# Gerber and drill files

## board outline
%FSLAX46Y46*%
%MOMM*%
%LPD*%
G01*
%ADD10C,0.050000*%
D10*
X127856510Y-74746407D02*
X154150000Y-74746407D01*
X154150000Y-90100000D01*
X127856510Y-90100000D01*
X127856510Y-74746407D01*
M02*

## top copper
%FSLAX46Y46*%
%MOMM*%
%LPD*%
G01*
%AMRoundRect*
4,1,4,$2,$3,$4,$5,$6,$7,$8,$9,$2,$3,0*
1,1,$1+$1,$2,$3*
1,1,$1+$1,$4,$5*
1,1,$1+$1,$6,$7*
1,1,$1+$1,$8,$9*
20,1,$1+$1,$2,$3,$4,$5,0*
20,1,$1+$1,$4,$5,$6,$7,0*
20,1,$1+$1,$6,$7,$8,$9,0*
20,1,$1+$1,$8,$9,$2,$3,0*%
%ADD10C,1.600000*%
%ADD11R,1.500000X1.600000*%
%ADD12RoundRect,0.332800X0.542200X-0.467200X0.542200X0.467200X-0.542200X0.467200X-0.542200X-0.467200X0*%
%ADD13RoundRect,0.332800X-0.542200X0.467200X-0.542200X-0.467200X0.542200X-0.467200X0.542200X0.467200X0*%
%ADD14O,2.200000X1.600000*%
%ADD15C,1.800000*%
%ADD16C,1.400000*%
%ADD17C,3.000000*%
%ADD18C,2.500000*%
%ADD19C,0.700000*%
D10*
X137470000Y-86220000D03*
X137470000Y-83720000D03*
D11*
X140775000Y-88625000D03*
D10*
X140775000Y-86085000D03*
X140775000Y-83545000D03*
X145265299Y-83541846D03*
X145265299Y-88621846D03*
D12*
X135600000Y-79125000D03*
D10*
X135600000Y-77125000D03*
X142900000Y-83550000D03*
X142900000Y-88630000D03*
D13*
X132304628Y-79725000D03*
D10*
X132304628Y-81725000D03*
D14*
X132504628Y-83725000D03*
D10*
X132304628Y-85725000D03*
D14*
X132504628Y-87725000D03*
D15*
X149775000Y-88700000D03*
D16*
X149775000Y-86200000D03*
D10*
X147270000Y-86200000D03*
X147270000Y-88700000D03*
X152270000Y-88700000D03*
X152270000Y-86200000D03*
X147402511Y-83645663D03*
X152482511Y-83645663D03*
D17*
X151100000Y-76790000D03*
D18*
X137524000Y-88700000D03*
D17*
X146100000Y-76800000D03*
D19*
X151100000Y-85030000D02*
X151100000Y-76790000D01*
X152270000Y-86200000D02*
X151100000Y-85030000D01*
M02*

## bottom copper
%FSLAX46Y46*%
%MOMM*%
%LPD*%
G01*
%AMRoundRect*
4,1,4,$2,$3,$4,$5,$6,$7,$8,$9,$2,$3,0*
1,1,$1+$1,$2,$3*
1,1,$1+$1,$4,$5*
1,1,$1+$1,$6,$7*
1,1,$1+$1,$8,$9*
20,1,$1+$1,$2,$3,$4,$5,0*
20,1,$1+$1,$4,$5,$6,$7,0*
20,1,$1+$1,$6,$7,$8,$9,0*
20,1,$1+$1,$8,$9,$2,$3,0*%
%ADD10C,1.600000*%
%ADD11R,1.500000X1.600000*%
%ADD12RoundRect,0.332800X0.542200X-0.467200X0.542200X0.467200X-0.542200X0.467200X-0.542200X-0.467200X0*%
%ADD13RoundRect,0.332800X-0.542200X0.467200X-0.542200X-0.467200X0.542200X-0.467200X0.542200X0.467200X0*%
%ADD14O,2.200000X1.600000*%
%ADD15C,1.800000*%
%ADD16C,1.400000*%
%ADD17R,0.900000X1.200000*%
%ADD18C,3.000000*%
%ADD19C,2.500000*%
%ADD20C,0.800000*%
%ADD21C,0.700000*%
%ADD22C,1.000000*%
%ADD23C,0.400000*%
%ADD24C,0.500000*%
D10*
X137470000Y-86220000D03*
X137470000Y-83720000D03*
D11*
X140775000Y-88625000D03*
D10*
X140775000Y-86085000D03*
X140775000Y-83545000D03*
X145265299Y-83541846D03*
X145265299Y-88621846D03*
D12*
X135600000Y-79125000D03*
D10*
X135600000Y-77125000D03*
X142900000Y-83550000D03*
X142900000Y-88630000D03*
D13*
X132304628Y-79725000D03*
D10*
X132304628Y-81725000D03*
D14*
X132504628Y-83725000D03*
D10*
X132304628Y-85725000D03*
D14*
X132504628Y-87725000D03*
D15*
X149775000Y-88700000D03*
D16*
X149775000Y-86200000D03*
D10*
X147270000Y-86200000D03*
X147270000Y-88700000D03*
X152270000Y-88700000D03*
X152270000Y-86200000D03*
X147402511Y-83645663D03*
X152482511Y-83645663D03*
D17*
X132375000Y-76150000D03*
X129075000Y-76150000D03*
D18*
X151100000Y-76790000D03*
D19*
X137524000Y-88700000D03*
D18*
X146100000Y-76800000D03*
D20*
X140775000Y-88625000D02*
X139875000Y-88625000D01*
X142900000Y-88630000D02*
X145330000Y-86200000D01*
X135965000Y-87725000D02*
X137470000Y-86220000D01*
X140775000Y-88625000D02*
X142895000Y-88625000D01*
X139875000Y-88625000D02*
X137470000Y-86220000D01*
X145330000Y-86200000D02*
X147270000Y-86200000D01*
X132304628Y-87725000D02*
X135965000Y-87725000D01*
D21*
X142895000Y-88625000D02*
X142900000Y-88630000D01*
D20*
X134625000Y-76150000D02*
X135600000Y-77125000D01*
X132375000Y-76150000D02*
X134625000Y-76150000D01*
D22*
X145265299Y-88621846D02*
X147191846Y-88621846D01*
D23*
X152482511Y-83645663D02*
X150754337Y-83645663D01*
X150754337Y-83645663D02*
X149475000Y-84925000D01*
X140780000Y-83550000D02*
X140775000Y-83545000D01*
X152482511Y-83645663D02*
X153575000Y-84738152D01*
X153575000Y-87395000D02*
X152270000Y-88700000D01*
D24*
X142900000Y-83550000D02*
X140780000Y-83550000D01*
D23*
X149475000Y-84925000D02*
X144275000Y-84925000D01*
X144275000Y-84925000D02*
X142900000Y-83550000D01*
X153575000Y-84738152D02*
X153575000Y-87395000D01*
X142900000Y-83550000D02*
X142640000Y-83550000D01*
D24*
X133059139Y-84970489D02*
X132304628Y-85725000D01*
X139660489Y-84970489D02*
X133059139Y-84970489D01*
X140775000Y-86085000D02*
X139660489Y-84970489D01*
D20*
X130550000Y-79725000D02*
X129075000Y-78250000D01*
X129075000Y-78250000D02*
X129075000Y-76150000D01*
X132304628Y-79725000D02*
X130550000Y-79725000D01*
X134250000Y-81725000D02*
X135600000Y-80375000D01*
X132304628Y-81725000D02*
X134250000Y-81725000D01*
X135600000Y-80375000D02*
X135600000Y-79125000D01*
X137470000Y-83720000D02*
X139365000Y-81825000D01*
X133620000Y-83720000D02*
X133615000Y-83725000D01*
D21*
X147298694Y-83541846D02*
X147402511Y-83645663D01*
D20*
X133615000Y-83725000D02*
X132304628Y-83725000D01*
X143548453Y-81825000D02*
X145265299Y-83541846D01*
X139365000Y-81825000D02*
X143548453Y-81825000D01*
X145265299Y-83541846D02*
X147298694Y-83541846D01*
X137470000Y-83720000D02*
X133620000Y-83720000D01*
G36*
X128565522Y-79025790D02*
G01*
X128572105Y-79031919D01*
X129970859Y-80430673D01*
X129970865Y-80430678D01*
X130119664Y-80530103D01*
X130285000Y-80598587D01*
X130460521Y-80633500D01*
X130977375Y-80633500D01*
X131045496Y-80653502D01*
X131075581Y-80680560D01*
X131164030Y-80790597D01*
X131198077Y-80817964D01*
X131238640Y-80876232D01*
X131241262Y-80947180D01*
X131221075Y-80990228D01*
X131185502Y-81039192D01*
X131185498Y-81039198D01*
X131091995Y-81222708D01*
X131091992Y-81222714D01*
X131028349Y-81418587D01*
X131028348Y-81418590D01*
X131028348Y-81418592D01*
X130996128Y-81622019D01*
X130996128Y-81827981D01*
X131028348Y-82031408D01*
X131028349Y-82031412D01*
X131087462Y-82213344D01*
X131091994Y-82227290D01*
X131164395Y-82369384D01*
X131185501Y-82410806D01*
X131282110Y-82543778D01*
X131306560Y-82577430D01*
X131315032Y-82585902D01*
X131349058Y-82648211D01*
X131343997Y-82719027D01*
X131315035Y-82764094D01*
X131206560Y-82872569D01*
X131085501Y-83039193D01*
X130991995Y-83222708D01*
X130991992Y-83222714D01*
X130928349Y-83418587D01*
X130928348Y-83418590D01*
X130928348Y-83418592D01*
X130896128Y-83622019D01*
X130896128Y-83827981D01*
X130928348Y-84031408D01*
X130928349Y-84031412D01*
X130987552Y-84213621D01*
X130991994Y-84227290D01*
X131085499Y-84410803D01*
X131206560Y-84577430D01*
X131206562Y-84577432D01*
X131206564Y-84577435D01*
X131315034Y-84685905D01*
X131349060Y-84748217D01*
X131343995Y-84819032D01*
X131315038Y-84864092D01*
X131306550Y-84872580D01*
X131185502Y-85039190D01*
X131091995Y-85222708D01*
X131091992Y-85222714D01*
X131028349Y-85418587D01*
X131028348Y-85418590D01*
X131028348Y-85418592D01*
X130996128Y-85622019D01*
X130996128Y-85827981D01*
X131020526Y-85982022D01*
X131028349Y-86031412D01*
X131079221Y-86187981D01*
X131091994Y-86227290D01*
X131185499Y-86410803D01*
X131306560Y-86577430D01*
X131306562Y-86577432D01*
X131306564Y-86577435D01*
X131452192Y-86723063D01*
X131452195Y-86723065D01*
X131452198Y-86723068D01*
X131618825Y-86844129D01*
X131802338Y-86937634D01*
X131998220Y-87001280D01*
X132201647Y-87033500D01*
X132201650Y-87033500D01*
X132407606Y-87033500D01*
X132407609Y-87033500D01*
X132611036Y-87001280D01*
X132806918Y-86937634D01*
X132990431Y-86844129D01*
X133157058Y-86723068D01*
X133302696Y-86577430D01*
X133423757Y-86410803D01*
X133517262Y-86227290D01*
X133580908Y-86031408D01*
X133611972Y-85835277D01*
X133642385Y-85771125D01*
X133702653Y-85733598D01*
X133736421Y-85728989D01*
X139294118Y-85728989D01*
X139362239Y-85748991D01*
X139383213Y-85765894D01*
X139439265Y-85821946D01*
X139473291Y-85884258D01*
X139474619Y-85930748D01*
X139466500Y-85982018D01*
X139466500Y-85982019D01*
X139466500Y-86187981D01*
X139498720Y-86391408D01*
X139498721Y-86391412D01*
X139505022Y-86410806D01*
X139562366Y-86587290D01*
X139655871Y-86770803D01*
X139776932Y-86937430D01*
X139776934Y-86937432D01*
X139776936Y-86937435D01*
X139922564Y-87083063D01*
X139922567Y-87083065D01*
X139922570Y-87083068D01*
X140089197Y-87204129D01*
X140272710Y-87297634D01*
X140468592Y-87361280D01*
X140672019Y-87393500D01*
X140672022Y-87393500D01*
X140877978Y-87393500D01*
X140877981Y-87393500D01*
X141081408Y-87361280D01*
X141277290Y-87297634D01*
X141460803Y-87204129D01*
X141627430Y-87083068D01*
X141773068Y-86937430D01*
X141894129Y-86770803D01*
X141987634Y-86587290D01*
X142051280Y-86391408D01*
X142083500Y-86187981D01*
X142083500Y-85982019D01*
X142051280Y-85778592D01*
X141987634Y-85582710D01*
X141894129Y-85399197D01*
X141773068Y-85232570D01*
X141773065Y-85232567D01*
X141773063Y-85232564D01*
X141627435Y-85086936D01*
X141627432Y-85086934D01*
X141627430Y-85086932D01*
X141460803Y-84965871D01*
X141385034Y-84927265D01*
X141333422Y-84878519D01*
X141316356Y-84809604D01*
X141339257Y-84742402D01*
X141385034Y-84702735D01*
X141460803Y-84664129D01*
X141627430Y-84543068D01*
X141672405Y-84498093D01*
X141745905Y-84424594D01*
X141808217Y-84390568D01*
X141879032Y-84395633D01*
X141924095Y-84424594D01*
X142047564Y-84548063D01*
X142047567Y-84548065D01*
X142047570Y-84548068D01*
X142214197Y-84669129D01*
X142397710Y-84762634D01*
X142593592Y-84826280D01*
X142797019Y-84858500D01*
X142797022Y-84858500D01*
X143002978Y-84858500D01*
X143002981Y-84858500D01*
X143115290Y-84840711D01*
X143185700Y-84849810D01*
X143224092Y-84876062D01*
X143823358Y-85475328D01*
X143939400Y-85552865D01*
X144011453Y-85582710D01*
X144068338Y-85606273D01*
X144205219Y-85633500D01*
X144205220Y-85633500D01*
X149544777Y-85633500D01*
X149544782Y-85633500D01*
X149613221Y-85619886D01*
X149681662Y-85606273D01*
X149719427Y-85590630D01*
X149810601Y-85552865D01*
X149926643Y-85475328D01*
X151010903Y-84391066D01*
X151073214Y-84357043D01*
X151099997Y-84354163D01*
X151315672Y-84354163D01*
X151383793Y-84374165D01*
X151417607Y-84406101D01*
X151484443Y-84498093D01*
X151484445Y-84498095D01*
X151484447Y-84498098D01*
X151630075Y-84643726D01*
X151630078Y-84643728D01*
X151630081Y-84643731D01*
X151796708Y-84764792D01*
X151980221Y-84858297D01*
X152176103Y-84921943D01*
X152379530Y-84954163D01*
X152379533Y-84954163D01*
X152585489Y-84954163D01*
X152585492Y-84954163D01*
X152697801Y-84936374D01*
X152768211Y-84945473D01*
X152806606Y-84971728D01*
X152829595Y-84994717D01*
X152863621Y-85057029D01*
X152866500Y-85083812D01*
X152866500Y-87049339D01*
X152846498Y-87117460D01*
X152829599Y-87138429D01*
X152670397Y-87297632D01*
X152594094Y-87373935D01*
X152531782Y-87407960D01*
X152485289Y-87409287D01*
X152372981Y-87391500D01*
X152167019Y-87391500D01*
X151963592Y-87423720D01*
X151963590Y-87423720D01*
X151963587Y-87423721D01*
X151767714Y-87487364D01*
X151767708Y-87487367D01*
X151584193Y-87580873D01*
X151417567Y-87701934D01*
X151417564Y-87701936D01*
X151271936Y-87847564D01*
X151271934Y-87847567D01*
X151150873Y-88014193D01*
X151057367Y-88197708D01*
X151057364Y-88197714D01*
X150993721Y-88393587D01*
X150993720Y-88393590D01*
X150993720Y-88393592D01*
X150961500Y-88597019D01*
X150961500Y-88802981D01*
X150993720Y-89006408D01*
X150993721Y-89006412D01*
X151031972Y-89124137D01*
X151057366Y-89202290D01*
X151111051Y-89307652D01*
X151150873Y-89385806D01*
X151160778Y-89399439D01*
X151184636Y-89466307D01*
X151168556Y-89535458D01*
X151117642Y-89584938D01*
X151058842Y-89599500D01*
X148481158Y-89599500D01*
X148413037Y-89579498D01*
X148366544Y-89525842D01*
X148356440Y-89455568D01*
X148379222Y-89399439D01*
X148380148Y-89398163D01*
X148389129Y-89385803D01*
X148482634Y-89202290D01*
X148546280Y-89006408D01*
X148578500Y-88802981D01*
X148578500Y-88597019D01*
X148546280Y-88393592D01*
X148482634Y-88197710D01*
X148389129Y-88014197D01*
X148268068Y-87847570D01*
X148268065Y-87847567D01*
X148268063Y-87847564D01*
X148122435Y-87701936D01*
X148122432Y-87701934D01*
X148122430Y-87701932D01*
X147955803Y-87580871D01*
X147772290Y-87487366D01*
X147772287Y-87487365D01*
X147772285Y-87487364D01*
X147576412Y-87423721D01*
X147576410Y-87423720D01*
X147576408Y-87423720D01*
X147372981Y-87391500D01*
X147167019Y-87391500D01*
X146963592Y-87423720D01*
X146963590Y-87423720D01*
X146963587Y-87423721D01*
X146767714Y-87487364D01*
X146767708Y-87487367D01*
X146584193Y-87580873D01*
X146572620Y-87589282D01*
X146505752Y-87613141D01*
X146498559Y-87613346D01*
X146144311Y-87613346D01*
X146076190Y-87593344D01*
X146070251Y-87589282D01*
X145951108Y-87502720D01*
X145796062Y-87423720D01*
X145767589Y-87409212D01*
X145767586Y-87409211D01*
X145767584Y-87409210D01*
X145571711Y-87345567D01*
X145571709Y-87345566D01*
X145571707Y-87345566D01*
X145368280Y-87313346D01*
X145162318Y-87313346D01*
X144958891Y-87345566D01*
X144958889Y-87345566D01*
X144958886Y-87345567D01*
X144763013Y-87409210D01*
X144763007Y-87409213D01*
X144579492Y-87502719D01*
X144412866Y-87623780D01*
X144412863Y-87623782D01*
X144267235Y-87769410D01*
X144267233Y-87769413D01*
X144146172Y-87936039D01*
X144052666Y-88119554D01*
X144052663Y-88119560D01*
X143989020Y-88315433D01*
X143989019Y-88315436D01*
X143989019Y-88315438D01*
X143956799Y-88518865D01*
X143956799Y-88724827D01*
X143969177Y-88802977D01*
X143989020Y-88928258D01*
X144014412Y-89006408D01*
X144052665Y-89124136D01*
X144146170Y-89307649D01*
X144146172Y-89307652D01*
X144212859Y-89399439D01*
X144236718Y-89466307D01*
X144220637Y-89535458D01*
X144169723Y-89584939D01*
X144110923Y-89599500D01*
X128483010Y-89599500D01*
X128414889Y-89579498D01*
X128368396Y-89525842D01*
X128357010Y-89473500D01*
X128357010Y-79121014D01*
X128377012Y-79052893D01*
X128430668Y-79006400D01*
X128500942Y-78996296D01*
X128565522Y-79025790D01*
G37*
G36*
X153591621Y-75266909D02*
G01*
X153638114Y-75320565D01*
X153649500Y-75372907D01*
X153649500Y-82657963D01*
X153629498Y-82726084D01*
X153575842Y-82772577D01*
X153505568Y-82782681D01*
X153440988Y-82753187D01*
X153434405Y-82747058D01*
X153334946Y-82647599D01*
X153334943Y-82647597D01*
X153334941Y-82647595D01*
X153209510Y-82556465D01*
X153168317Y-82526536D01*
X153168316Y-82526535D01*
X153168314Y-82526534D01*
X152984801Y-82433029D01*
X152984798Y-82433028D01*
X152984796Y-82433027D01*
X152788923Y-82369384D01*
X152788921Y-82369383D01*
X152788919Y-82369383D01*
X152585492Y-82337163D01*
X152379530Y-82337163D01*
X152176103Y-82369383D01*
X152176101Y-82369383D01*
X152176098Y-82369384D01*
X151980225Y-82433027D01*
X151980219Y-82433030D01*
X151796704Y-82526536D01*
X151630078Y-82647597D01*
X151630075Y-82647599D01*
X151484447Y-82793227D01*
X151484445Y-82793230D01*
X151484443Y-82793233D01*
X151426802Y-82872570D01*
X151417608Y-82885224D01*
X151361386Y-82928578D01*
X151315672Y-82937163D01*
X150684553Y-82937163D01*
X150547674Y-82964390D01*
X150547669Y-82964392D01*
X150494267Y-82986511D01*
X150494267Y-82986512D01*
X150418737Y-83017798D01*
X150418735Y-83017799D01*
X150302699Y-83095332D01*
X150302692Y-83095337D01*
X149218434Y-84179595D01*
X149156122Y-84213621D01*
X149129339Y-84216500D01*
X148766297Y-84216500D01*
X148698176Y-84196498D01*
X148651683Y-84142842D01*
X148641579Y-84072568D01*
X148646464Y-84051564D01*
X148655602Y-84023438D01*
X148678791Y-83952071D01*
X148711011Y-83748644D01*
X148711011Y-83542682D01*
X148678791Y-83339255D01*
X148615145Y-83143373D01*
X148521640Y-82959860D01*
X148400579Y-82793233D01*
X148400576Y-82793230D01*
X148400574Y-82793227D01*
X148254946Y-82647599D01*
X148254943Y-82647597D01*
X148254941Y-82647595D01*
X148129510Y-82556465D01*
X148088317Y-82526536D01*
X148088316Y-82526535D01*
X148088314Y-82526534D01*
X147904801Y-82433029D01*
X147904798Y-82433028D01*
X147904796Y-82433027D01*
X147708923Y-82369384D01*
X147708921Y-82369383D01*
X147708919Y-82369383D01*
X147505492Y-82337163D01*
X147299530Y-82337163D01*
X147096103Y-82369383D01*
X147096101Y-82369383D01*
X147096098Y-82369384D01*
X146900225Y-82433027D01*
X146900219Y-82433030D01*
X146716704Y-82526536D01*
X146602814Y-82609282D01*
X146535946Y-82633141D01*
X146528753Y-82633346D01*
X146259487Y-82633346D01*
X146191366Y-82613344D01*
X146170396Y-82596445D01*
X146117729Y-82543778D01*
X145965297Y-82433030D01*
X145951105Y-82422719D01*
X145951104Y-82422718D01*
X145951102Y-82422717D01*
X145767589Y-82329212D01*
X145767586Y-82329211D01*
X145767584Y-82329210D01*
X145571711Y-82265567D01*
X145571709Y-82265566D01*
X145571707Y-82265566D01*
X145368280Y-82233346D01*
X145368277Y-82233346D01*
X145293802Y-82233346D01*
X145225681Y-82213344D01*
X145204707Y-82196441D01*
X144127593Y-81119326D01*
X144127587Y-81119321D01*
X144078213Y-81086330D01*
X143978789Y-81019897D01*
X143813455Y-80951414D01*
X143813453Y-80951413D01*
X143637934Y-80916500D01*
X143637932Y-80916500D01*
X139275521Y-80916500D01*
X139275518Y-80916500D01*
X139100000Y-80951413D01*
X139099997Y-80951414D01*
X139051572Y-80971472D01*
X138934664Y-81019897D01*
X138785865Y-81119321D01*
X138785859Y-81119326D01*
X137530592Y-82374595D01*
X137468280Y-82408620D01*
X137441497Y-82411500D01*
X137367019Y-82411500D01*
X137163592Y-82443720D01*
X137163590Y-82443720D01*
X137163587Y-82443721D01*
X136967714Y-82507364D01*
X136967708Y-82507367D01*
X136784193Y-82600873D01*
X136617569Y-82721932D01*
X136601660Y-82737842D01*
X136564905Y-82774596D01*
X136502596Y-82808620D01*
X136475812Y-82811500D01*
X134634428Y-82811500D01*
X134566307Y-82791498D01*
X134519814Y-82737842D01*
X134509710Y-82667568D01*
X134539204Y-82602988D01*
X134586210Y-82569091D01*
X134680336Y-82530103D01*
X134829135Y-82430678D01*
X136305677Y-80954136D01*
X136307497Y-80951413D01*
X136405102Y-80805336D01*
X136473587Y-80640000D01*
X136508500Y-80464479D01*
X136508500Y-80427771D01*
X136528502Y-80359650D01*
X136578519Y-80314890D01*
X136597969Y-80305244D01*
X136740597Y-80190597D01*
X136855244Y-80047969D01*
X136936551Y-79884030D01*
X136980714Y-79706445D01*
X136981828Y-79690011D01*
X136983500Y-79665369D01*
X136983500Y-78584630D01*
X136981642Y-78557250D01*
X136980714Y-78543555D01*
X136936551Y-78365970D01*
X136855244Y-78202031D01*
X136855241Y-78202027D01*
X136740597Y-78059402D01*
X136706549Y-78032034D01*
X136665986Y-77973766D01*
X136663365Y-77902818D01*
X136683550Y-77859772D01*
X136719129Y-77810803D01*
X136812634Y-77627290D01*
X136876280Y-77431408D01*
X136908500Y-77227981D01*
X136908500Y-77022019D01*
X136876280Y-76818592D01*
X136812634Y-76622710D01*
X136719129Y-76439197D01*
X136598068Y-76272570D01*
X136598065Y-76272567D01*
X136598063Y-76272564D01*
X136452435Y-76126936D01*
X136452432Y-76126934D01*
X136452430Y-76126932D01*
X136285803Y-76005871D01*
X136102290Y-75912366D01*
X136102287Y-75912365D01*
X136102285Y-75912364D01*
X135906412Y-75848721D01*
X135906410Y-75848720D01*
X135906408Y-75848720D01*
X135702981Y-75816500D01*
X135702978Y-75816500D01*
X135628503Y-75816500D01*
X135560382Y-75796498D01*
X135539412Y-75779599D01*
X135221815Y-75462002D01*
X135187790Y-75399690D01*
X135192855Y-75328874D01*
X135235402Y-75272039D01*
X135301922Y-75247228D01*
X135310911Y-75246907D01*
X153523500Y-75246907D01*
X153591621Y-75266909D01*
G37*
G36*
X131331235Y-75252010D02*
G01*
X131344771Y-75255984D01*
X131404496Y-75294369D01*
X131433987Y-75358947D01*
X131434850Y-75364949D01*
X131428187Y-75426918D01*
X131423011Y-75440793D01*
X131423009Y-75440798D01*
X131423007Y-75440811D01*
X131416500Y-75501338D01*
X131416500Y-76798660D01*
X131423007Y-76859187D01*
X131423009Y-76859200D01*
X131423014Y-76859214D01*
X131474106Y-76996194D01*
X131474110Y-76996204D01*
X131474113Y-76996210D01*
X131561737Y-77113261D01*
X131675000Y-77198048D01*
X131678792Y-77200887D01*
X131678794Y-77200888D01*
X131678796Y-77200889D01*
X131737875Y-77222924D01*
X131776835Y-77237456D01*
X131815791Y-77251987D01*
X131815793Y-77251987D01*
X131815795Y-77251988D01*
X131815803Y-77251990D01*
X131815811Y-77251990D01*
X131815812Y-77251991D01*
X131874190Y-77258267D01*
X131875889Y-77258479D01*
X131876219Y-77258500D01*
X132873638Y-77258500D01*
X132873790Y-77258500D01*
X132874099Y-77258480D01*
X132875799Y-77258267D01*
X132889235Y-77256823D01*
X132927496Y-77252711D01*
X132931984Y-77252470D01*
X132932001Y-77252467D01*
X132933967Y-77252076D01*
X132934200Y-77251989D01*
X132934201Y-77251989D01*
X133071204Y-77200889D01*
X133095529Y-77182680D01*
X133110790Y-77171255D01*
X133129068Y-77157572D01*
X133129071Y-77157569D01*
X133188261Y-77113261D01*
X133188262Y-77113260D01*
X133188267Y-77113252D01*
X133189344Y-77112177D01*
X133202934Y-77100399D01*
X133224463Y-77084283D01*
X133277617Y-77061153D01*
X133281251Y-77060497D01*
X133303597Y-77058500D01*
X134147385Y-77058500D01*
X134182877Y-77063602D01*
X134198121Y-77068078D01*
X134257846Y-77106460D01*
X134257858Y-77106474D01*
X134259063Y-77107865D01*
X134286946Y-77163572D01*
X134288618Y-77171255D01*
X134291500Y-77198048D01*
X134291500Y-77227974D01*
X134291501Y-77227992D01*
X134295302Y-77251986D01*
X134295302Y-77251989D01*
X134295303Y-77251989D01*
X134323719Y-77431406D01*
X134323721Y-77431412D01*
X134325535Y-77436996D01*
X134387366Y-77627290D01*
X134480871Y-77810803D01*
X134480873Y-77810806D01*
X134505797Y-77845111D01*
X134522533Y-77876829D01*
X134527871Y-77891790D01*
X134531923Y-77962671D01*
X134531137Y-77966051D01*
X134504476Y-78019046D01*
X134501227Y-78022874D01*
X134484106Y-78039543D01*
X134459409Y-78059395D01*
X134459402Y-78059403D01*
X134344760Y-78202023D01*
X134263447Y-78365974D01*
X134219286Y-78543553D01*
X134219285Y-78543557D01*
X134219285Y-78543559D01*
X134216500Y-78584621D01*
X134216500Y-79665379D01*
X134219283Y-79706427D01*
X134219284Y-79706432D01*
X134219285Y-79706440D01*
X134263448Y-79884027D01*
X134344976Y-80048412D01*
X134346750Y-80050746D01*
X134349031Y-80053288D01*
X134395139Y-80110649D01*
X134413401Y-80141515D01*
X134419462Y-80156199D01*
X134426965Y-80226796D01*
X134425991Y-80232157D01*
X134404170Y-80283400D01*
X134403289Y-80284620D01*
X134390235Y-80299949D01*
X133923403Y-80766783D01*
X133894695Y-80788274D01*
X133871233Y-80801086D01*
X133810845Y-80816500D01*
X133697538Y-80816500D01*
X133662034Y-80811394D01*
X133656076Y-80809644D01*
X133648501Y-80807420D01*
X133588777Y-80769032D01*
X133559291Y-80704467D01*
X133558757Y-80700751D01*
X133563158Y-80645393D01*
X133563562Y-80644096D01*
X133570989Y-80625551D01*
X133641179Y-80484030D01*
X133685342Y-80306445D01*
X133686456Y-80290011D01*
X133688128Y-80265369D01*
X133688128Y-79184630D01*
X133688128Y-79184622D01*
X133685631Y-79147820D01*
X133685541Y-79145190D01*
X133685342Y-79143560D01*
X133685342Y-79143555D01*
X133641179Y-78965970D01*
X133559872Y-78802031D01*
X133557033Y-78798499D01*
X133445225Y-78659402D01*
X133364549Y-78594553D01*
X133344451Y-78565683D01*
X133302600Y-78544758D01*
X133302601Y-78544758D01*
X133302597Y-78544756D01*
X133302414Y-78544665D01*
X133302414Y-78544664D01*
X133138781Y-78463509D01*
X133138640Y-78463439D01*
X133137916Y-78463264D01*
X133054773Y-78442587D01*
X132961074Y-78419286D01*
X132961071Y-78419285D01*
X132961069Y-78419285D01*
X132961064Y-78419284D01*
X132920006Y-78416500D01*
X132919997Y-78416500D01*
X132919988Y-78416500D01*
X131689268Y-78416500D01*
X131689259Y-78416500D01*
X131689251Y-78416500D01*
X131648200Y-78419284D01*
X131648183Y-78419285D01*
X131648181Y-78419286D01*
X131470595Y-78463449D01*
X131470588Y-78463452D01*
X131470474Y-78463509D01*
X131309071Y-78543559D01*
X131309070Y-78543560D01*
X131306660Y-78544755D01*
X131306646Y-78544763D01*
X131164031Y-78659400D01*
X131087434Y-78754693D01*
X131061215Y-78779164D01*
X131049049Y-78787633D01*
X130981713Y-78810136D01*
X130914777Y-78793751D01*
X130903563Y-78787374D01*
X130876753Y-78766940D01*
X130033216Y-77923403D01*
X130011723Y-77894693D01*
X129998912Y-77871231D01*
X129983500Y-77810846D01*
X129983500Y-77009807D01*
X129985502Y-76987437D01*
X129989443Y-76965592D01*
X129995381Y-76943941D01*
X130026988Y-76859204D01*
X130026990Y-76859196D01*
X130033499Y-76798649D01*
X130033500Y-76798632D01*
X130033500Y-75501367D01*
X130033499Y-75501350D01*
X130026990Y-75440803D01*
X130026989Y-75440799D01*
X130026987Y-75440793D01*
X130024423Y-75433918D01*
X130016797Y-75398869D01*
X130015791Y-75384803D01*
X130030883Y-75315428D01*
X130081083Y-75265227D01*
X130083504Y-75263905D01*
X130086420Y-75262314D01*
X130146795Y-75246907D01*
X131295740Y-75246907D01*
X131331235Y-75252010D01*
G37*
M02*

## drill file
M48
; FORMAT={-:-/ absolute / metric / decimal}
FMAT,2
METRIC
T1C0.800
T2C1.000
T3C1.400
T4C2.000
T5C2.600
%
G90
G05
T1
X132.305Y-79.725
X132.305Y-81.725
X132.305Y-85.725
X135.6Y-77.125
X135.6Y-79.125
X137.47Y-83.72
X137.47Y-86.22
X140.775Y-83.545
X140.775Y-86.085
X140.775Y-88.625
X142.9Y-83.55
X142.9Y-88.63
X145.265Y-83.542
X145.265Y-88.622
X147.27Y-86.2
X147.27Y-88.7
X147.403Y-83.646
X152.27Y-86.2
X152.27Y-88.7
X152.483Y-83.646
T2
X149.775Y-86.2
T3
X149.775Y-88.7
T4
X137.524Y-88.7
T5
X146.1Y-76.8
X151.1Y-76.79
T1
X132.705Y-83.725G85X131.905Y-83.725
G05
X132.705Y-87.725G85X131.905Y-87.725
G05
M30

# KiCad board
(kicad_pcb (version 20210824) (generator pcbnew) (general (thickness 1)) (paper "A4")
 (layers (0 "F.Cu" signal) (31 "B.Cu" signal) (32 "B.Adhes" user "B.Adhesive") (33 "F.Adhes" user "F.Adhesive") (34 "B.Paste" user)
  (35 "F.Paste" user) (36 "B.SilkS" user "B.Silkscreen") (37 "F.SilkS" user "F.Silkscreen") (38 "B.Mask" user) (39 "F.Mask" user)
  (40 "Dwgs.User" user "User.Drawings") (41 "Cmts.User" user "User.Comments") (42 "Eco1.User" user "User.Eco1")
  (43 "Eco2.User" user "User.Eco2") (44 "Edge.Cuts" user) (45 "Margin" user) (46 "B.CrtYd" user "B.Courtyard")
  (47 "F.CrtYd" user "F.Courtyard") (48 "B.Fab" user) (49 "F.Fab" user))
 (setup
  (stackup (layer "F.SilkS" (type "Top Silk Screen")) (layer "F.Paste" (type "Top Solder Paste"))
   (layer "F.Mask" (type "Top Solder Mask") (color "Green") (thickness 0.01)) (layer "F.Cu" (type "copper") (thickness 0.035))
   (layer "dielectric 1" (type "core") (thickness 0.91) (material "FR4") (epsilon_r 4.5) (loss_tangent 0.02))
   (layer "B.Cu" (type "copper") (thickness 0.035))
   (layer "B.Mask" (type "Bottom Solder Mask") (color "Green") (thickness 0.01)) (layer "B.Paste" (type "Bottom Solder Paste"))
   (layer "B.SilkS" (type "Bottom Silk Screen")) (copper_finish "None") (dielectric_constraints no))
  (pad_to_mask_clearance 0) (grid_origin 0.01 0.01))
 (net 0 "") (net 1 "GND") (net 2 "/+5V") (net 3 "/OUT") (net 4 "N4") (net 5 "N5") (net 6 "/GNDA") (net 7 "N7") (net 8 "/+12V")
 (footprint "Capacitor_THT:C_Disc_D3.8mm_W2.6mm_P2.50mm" (layer "F.Cu") (at 137.47 86.22 90)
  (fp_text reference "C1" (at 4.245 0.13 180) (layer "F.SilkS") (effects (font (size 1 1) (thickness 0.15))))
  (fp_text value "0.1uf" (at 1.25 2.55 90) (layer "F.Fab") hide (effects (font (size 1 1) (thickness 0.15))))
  (pad "1" thru_hole circle locked (at 0 0 90) (size 1.6 1.6) (drill 0.8) (layers *.Cu *.Mask) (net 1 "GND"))
  (pad "2" thru_hole circle locked (at 2.5 0 90) (size 1.6 1.6) (drill 0.8) (layers *.Cu *.Mask) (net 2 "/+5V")))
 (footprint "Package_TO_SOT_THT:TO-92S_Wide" (layer "F.Cu") (at 140.775 88.625 90)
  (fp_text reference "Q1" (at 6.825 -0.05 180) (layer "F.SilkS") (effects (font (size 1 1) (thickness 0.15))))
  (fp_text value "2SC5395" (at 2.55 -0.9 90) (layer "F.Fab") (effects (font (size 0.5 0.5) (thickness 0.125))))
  (pad "1" thru_hole rect locked (at 0 0 90) (size 1.6 1.5) (drill 0.8) (layers *.Cu *.Mask) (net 1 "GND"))
  (pad "2" thru_hole circle locked (at 2.54 0 90) (size 1.6 1.6) (drill 0.8) (layers *.Cu *.Mask) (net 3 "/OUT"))
  (pad "3" thru_hole circle locked (at 5.08 0 90) (size 1.6 1.6) (drill 0.8) (layers *.Cu *.Mask) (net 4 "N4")))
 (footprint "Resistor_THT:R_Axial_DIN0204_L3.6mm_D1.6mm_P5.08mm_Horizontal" (layer "F.Cu") (at 145.265299 83.541846 -90)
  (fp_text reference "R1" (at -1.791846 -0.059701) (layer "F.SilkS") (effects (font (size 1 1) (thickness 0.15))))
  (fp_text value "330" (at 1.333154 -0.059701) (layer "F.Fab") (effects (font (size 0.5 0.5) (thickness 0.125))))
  (pad "1" thru_hole circle locked (at 0 0 270) (size 1.6 1.6) (drill 0.8) (layers *.Cu *.Mask) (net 2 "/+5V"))
  (pad "2" thru_hole circle locked (at 5.08 0 270) (size 1.6 1.6) (drill 0.8) (layers *.Cu *.Mask) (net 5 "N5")))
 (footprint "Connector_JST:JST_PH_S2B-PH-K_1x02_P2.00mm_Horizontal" (layer "F.Cu") (at 135.6 79.125 90)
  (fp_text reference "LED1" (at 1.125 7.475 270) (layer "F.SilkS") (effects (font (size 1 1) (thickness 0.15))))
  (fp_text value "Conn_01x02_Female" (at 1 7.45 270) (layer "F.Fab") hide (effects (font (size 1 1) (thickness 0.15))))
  (pad "1" thru_hole roundrect locked (at 0 0 90) (size 1.6 1.75) (drill 0.8) (layers *.Cu *.Mask) (roundrect_rratio 0.208) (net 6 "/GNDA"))
  (pad "2" thru_hole circle locked (at 2 0 90) (size 1.6 1.6) (drill 0.8) (layers *.Cu *.Mask) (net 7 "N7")))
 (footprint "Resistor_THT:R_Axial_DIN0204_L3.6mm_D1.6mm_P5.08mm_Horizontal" (layer "F.Cu") (at 142.9 83.55 -90)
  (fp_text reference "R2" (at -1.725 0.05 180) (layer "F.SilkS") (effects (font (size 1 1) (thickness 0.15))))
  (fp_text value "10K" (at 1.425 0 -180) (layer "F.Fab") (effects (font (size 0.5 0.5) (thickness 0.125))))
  (pad "1" thru_hole circle locked (at 0 0 270) (size 1.6 1.6) (drill 0.8) (layers *.Cu *.Mask) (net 4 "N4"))
  (pad "2" thru_hole circle locked (at 5.08 0 270) (size 1.6 1.6) (drill 0.8) (layers *.Cu *.Mask) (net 1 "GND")))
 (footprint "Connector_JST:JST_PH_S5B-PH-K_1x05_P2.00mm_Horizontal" (layer "F.Cu") (at 132.304628 79.725 -90)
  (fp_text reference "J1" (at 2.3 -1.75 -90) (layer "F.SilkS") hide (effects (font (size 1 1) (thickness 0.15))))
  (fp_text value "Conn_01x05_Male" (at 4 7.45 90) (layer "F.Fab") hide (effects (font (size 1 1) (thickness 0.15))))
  (pad "1" thru_hole roundrect locked (at 0 0 270) (size 1.6 1.75) (drill 0.8) (layers *.Cu *.Mask) (roundrect_rratio 0.208) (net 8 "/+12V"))
  (pad "2" thru_hole circle locked (at 2 0 270) (size 1.6 1.6) (drill 0.8) (layers *.Cu *.Mask) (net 6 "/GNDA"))
  (pad "3" thru_hole oval locked (at 4 0 270) (size 1.6 2.2) (drill oval 0.8 1.6 (offset 0 -0.2)) (layers *.Cu *.Mask) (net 2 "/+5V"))
  (pad "4" thru_hole circle locked (at 6 0 270) (size 1.6 1.6) (drill 0.8) (layers *.Cu *.Mask) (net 3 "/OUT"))
  (pad "5" thru_hole oval locked (at 8 0 270) (size 1.6 2.2) (drill oval 0.8 1.6 (offset 0 -0.2)) (layers *.Cu *.Mask) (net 1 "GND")))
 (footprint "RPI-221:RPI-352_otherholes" (layer "F.Cu") (at 149.775 86.18)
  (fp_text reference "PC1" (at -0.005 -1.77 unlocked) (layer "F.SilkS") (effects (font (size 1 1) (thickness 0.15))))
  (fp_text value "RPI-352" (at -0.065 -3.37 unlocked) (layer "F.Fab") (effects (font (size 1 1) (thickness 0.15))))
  (pad "" thru_hole circle (at 0 2.52) (size 1.8 1.8) (drill 1.4) (layers *.Cu *.Mask) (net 1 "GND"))
  (pad "" thru_hole circle (at 0 0.02) (size 1.4 1.4) (drill 1) (layers *.Cu *.Mask) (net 1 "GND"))
  (pad "1" thru_hole circle locked (at -2.505 0.02) (size 1.6 1.6) (drill 0.8) (layers *.Cu *.Mask) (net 1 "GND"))
  (pad "2" thru_hole circle locked (at -2.505 2.52) (size 1.6 1.6) (drill 0.8) (layers *.Cu *.Mask) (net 5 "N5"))
  (pad "3" thru_hole circle locked (at 2.495 2.52) (size 1.6 1.6) (drill 0.8) (layers *.Cu *.Mask) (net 4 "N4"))
  (pad "4" thru_hole circle locked (at 2.495 0.02) (size 1.6 1.6) (drill 0.8) (layers *.Cu *.Mask) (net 1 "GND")))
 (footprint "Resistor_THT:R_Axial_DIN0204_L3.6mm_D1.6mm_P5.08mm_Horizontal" (layer "F.Cu") (at 147.402511 83.645663)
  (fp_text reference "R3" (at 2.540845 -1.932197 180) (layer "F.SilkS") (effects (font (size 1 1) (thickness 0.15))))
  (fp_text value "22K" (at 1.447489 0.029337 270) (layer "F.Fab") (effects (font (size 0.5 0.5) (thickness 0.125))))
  (pad "1" thru_hole circle locked (at 0 0) (size 1.6 1.6) (drill 0.8) (layers *.Cu *.Mask) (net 2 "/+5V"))
  (pad "2" thru_hole circle locked (at 5.08 0) (size 1.6 1.6) (drill 0.8) (layers *.Cu *.Mask) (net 4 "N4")))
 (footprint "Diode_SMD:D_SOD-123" (layer "B.Cu") (at 130.725 76.15 180)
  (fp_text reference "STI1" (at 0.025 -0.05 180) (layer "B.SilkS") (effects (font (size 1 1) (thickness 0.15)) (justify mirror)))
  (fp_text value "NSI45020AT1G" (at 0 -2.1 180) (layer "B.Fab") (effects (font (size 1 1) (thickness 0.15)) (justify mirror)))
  (pad "1" smd rect locked (at -1.65 0 180) (size 0.9 1.2) (layers "B.Cu" "B.Paste" "B.Mask") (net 7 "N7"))
  (pad "2" smd rect locked (at 1.65 0 180) (size 0.9 1.2) (layers "B.Cu" "B.Paste" "B.Mask") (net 8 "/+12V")))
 (gr_rect (start 127.85651 74.746407) (end 154.15 90.1) (layer "Edge.Cuts") (width 0.05) (fill none))
 (segment (start 151.1 85.03) (end 151.1 76.79) (width 0.7) (layer "F.Cu") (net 1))
 (segment (start 152.27 86.2) (end 151.1 85.03) (width 0.7) (layer "F.Cu") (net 1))
 (via (at 151.1 76.79) (size 3) (drill 2.6) (layers "F.Cu" "B.Cu") (free) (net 1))
 (via (at 137.524 88.7) (size 2.5) (drill 2) (layers "F.Cu" "B.Cu") (free) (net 1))
 (via (at 146.1 76.8) (size 3) (drill 2.6) (layers "F.Cu" "B.Cu") (free) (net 1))
 (segment (start 140.775 88.625) (end 139.875 88.625) (width 0.8) (layer "B.Cu") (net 1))
 (segment (start 142.9 88.63) (end 145.33 86.2) (width 0.8) (layer "B.Cu") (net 1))
 (segment (start 135.965 87.725) (end 137.47 86.22) (width 0.8) (layer "B.Cu") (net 1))
 (segment (start 140.775 88.625) (end 142.895 88.625) (width 0.8) (layer "B.Cu") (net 1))
 (segment (start 139.875 88.625) (end 137.47 86.22) (width 0.8) (layer "B.Cu") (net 1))
 (segment (start 145.33 86.2) (end 147.27 86.2) (width 0.8) (layer "B.Cu") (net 1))
 (segment (start 132.304628 87.725) (end 135.965 87.725) (width 0.8) (layer "B.Cu") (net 1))
 (segment (start 142.895 88.625) (end 142.9 88.63) (width 0.7) (layer "B.Cu") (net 1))
 (segment (start 134.625 76.15) (end 135.6 77.125) (width 0.8) (layer "B.Cu") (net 7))
 (segment (start 132.375 76.15) (end 134.625 76.15) (width 0.8) (layer "B.Cu") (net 7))
 (segment (start 145.265299 88.621846) (end 147.191846 88.621846) (width 1) (layer "B.Cu") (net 5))
 (segment (start 152.482511 83.645663) (end 150.754337 83.645663) (width 0.4) (layer "B.Cu") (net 4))
 (segment (start 150.754337 83.645663) (end 149.475 84.925) (width 0.4) (layer "B.Cu") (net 4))
 (segment (start 140.78 83.55) (end 140.775 83.545) (width 0.4) (layer "B.Cu") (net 4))
 (segment (start 152.482511 83.645663) (end 153.575 84.738152) (width 0.4) (layer "B.Cu") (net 4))
 (segment (start 153.575 87.395) (end 152.27 88.7) (width 0.4) (layer "B.Cu") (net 4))
 (segment (start 142.9 83.55) (end 140.78 83.55) (width 0.5) (layer "B.Cu") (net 4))
 (segment (start 149.475 84.925) (end 144.275 84.925) (width 0.4) (layer "B.Cu") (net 4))
 (segment (start 144.275 84.925) (end 142.9 83.55) (width 0.4) (layer "B.Cu") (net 4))
 (segment (start 153.575 84.738152) (end 153.575 87.395) (width 0.4) (layer "B.Cu") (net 4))
 (segment (start 142.9 83.55) (end 142.64 83.55) (width 0.4) (layer "B.Cu") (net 4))
 (segment (start 133.059139 84.970489) (end 132.304628 85.725) (width 0.5) (layer "B.Cu") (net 3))
 (segment (start 139.660489 84.970489) (end 133.059139 84.970489) (width 0.5) (layer "B.Cu") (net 3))
 (segment (start 140.775 86.085) (end 139.660489 84.970489) (width 0.5) (layer "B.Cu") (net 3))
 (segment (start 130.55 79.725) (end 129.075 78.25) (width 0.8) (layer "B.Cu") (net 8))
 (segment (start 129.075 78.25) (end 129.075 76.15) (width 0.8) (layer "B.Cu") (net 8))
 (segment (start 132.304628 79.725) (end 130.55 79.725) (width 0.8) (layer "B.Cu") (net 8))
 (segment (start 134.25 81.725) (end 135.6 80.375) (width 0.8) (layer "B.Cu") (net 6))
 (segment (start 132.304628 81.725) (end 134.25 81.725) (width 0.8) (layer "B.Cu") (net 6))
 (segment (start 135.6 80.375) (end 135.6 79.125) (width 0.8) (layer "B.Cu") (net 6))
 (segment (start 137.47 83.72) (end 139.365 81.825) (width 0.8) (layer "B.Cu") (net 2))
 (segment (start 133.62 83.72) (end 133.615 83.725) (width 0.8) (layer "B.Cu") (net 2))
 (segment (start 147.298694 83.541846) (end 147.402511 83.645663) (width 0.7) (layer "B.Cu") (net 2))
 (segment (start 133.615 83.725) (end 132.304628 83.725) (width 0.8) (layer "B.Cu") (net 2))
 (segment (start 143.548453 81.825) (end 145.265299 83.541846) (width 0.8) (layer "B.Cu") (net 2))
 (segment (start 139.365 81.825) (end 143.548453 81.825) (width 0.8) (layer "B.Cu") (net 2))
 (segment (start 145.265299 83.541846) (end 147.298694 83.541846) (width 0.8) (layer "B.Cu") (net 2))
 (segment (start 137.47 83.72) (end 133.62 83.72) (width 0.8) (layer "B.Cu") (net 2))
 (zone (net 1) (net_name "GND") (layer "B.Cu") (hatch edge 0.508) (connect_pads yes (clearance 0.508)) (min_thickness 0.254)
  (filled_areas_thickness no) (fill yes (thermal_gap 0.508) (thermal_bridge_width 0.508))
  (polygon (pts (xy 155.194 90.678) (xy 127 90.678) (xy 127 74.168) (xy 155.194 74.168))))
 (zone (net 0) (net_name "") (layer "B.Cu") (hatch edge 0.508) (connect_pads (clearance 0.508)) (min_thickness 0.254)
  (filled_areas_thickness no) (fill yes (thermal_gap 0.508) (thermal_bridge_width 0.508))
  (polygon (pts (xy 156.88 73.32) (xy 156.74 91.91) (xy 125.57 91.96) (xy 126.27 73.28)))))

